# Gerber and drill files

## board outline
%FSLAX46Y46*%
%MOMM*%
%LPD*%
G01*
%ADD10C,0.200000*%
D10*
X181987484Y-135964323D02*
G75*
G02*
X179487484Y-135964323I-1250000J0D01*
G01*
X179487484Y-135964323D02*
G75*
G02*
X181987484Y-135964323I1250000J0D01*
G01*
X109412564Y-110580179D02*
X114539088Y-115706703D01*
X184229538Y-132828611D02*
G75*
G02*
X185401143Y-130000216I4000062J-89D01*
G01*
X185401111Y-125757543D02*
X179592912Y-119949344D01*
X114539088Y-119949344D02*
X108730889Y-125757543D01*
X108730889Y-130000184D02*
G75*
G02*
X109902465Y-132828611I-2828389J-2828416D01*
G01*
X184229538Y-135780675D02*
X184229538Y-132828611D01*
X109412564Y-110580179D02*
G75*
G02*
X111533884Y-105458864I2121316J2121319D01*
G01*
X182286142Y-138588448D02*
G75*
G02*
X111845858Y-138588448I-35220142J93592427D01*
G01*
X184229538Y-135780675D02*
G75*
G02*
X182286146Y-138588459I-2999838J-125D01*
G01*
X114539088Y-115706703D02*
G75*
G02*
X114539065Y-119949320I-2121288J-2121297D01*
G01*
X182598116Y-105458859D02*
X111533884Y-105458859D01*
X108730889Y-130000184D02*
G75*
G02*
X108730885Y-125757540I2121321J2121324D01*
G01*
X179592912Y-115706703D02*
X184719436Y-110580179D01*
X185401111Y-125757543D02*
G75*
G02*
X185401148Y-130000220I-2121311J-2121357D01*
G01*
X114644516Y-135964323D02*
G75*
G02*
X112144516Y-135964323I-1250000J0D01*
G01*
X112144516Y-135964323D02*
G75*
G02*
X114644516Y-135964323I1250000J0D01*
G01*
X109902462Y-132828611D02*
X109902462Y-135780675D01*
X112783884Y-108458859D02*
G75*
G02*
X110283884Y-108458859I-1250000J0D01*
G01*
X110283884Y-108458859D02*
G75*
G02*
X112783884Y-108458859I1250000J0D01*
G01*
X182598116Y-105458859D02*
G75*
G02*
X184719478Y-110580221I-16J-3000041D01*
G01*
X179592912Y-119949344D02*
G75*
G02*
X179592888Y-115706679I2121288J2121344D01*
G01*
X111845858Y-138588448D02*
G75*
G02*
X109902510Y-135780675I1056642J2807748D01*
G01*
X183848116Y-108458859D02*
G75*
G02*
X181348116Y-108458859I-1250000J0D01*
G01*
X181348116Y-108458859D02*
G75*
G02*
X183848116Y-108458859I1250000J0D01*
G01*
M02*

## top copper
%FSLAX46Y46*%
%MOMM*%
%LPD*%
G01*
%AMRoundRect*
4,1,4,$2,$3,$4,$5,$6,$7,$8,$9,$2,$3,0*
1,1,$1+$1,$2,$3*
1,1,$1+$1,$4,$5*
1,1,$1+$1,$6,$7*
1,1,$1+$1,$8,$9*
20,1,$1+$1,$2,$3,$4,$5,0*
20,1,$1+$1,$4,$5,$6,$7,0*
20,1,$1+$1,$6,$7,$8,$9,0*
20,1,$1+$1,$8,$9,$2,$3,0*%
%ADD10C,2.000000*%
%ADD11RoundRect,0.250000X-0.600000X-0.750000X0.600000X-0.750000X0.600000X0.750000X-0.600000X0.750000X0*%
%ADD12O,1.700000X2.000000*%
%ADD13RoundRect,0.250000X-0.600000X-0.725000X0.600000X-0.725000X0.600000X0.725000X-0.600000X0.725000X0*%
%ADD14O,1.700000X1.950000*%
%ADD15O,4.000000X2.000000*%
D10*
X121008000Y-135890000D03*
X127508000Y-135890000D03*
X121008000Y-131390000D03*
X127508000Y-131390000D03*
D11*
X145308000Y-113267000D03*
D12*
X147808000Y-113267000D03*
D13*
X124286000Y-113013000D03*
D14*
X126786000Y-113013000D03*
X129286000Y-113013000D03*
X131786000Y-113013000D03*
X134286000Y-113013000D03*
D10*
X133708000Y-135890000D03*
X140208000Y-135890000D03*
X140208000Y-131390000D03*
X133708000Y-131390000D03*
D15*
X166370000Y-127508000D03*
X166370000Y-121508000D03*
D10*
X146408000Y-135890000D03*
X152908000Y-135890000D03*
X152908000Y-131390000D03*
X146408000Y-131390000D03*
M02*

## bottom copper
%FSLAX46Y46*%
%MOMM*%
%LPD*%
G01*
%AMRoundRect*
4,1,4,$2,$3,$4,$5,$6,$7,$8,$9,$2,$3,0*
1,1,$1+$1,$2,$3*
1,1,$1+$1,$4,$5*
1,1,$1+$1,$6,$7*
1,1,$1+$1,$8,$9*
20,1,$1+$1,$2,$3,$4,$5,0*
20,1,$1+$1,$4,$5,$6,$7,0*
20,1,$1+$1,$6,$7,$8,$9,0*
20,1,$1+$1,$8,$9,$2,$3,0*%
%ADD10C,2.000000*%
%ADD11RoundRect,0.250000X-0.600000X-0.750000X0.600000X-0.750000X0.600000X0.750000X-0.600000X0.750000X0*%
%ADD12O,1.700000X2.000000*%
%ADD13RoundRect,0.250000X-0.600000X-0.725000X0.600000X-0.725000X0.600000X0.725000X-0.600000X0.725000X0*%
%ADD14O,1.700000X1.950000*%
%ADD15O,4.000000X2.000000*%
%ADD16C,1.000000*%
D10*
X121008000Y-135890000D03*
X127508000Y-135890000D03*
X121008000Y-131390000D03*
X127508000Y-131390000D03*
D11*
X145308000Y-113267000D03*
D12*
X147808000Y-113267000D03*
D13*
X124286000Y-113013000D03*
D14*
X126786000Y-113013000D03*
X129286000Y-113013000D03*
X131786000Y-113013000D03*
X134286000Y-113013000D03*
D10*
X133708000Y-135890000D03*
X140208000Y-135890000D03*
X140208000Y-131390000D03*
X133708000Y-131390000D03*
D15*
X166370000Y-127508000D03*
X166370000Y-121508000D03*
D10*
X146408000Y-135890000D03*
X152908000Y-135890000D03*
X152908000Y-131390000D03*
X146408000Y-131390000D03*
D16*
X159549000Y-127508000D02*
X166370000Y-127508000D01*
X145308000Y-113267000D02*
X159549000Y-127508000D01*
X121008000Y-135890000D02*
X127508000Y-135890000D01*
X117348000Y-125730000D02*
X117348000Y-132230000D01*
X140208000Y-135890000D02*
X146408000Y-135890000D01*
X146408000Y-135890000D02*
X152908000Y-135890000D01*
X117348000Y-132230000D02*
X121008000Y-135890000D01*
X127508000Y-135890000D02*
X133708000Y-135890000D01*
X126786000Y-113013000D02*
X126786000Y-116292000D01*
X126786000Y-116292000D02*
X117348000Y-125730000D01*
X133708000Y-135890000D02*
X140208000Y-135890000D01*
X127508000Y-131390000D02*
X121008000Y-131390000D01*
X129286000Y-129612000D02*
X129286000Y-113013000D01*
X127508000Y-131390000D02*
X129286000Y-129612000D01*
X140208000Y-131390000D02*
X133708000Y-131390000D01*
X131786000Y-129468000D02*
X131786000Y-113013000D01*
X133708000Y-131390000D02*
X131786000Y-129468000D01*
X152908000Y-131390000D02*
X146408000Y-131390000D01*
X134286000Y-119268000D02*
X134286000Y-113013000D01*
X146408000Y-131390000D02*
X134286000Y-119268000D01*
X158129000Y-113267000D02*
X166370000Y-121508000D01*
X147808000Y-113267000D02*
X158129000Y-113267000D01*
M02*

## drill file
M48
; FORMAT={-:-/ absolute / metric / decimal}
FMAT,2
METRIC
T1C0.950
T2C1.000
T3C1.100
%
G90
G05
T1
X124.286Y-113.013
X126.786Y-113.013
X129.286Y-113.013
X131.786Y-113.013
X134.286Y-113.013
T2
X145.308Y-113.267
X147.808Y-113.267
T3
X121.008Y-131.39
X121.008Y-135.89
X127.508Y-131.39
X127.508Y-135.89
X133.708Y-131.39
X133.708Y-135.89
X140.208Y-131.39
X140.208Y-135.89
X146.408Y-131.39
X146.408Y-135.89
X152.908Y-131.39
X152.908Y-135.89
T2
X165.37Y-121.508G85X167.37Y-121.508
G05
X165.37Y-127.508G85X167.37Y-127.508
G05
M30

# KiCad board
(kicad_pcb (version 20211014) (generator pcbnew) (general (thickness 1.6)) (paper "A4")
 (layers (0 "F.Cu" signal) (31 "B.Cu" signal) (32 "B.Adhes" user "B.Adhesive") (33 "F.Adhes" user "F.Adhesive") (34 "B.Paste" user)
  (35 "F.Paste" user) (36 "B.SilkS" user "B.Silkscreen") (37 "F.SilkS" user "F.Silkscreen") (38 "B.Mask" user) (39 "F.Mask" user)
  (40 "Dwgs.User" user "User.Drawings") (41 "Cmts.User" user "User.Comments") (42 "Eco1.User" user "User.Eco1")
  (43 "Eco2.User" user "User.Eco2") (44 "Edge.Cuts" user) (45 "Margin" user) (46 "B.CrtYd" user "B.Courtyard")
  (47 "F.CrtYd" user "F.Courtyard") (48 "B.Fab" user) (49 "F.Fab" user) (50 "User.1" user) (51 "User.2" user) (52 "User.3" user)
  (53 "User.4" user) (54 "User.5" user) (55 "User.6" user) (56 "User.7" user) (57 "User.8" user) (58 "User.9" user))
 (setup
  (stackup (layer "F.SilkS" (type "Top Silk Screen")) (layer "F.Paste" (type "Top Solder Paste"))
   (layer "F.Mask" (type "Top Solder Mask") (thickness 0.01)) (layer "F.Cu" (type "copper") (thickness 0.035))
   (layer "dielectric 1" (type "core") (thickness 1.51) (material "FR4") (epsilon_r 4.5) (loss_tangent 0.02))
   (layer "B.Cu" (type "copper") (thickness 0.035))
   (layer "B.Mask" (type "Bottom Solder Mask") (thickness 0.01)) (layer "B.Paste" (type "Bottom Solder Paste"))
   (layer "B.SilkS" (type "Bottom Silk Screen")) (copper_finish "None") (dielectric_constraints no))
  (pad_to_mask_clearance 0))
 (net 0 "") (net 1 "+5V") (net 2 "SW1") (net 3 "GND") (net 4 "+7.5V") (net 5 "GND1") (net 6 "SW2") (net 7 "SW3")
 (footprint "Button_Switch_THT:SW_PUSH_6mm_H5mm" (layer "F.Cu") (at 127.508 135.89 180)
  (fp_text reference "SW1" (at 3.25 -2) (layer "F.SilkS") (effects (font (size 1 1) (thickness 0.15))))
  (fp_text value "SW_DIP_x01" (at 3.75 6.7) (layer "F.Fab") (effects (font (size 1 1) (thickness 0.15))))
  (pad "1" thru_hole circle (at 6.5 0 270) (size 2 2) (drill 1.1) (layers *.Cu *.Mask) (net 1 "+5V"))
  (pad "1" thru_hole circle (at 0 0 270) (size 2 2) (drill 1.1) (layers *.Cu *.Mask) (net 1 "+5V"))
  (pad "2" thru_hole circle (at 6.5 4.5 270) (size 2 2) (drill 1.1) (layers *.Cu *.Mask) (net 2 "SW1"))
  (pad "2" thru_hole circle (at 0 4.5 270) (size 2 2) (drill 1.1) (layers *.Cu *.Mask) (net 2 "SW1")))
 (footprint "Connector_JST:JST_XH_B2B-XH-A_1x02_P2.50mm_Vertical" (layer "F.Cu") (at 145.308 113.267)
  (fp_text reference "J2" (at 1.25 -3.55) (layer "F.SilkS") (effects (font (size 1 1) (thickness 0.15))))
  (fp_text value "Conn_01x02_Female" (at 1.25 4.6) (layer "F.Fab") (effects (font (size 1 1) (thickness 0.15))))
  (pad "1" thru_hole roundrect (at 0 0) (size 1.7 2) (drill 1) (layers *.Cu *.Mask) (roundrect_rratio 0.1470588235) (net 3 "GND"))
  (pad "2" thru_hole oval (at 2.5 0) (size 1.7 2) (drill 1) (layers *.Cu *.Mask) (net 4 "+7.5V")))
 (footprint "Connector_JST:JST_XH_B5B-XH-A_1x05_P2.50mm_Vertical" (layer "F.Cu") (at 124.286 113.013)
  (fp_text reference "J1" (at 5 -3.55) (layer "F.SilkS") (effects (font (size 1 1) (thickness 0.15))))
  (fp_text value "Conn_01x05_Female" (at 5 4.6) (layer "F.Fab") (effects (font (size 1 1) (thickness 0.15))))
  (pad "1" thru_hole roundrect (at 0 0) (size 1.7 1.95) (drill 0.95) (layers *.Cu *.Mask) (roundrect_rratio 0.1470588235) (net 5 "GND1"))
  (pad "2" thru_hole oval (at 2.5 0) (size 1.7 1.95) (drill 0.95) (layers *.Cu *.Mask) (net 1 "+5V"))
  (pad "3" thru_hole oval (at 5 0) (size 1.7 1.95) (drill 0.95) (layers *.Cu *.Mask) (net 2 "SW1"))
  (pad "4" thru_hole oval (at 7.5 0) (size 1.7 1.95) (drill 0.95) (layers *.Cu *.Mask) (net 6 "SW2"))
  (pad "5" thru_hole oval (at 10 0) (size 1.7 1.95) (drill 0.95) (layers *.Cu *.Mask) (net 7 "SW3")))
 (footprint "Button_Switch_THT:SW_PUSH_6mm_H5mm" (layer "F.Cu") (at 140.208 135.89 180)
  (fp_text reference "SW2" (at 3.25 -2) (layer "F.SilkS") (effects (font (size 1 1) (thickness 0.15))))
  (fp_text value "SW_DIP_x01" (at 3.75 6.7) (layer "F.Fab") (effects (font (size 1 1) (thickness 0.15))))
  (pad "1" thru_hole circle (at 6.5 0 270) (size 2 2) (drill 1.1) (layers *.Cu *.Mask) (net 1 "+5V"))
  (pad "1" thru_hole circle (at 0 0 270) (size 2 2) (drill 1.1) (layers *.Cu *.Mask) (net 1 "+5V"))
  (pad "2" thru_hole circle (at 0 4.5 270) (size 2 2) (drill 1.1) (layers *.Cu *.Mask) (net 6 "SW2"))
  (pad "2" thru_hole circle (at 6.5 4.5 270) (size 2 2) (drill 1.1) (layers *.Cu *.Mask) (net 6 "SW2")))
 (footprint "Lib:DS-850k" (layer "F.Cu") (at 166.37 127.508 -90)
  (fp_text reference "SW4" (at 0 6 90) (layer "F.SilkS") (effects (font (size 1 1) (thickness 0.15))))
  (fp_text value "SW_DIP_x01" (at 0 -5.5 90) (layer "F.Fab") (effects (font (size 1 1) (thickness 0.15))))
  (pad "1" thru_hole oval locked (at 0 0) (size 4 2) (drill oval 3 1) (layers *.Cu *.Mask) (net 3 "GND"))
  (pad "2" thru_hole oval locked (at -6 0) (size 4 2) (drill oval 3 1) (layers *.Cu *.Mask) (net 4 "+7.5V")))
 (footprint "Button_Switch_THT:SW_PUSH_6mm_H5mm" (layer "F.Cu") (at 152.908 135.89 180)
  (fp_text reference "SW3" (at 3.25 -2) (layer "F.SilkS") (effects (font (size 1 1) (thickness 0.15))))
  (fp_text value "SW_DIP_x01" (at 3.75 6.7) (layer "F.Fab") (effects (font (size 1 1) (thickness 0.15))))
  (pad "1" thru_hole circle (at 6.5 0 270) (size 2 2) (drill 1.1) (layers *.Cu *.Mask) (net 1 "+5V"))
  (pad "1" thru_hole circle (at 0 0 270) (size 2 2) (drill 1.1) (layers *.Cu *.Mask) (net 1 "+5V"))
  (pad "2" thru_hole circle (at 0 4.5 270) (size 2 2) (drill 1.1) (layers *.Cu *.Mask) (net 7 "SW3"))
  (pad "2" thru_hole circle (at 6.5 4.5 270) (size 2 2) (drill 1.1) (layers *.Cu *.Mask) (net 7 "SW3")))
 (gr_circle (center 180.737484 135.964323) (end 181.987484 135.964323) (layer "Edge.Cuts") (width 0.2) (fill none))
 (gr_line (start 109.412564 110.580179) (end 114.539088 115.706703) (layer "Edge.Cuts") (width 0.2))
 (gr_arc (start 184.229538 132.828611) (mid 184.534027 131.297882) (end 185.401111 130.000184) (layer "Edge.Cuts") (width 0.2))
 (gr_line (start 185.401111 125.757543) (end 179.592912 119.949344) (layer "Edge.Cuts") (width 0.2))
 (gr_line (start 114.539088 119.949344) (end 108.730889 125.757543) (layer "Edge.Cuts") (width 0.2))
 (gr_arc (start 108.730889 130.000184) (mid 109.59798 131.297877) (end 109.902462 132.828611) (layer "Edge.Cuts") (width 0.2))
 (gr_line (start 184.229538 135.780675) (end 184.229538 132.828611) (layer "Edge.Cuts") (width 0.2))
 (gr_arc (start 109.412564 110.580179) (mid 108.762246 107.310809) (end 111.533884 105.458859) (layer "Edge.Cuts") (width 0.2))
 (gr_arc (start 182.286142 138.588448) (mid 147.066 144.996025) (end 111.845858 138.588448) (layer "Edge.Cuts") (width 0.2))
 (gr_arc (start 184.229538 135.780675) (mid 183.696321 137.488069) (end 182.286142 138.588448) (layer "Edge.Cuts") (width 0.2))
 (gr_arc (start 114.539088 115.706703) (mid 115.417768 117.828024) (end 114.539088 119.949344) (layer "Edge.Cuts") (width 0.2))
 (gr_line (start 182.598116 105.458859) (end 111.533884 105.458859) (layer "Edge.Cuts") (width 0.2))
 (gr_arc (start 108.730889 130.000184) (mid 107.852209 127.878864) (end 108.730889 125.757543) (layer "Edge.Cuts") (width 0.2))
 (gr_line (start 179.592912 115.706703) (end 184.719436 110.580179) (layer "Edge.Cuts") (width 0.2))
 (gr_arc (start 185.401111 125.757543) (mid 186.279792 127.878864) (end 185.401111 130.000184) (layer "Edge.Cuts") (width 0.2))
 (gr_circle (center 113.394516 135.964323) (end 114.644516 135.964323) (layer "Edge.Cuts") (width 0.2) (fill none))
 (gr_line (start 109.902462 132.828611) (end 109.902462 135.780675) (layer "Edge.Cuts") (width 0.2))
 (gr_circle (center 111.533884 108.458859) (end 112.783884 108.458859) (layer "Edge.Cuts") (width 0.2) (fill none))
 (gr_arc (start 182.598116 105.458859) (mid 185.369755 107.310807) (end 184.719436 110.580179) (layer "Edge.Cuts") (width 0.2))
 (gr_arc (start 179.592912 119.949344) (mid 178.714233 117.828024) (end 179.592912 115.706703) (layer "Edge.Cuts") (width 0.2))
 (gr_arc (start 111.845858 138.588448) (mid 110.435702 137.48804) (end 109.902462 135.780675) (layer "Edge.Cuts") (width 0.2))
 (gr_circle (center 182.598116 108.458859) (end 183.848116 108.458859) (layer "Edge.Cuts") (width 0.2) (fill none))
 (segment (start 159.549 127.508) (end 166.37 127.508) (width 1) (layer "B.Cu") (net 3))
 (segment (start 145.308 113.267) (end 159.549 127.508) (width 1) (layer "B.Cu") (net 3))
 (segment (start 121.008 135.89) (end 127.508 135.89) (width 1) (layer "B.Cu") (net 1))
 (segment (start 117.348 125.73) (end 117.348 132.23) (width 1) (layer "B.Cu") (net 1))
 (segment (start 140.208 135.89) (end 146.408 135.89) (width 1) (layer "B.Cu") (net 1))
 (segment (start 146.408 135.89) (end 152.908 135.89) (width 1) (layer "B.Cu") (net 1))
 (segment (start 117.348 132.23) (end 121.008 135.89) (width 1) (layer "B.Cu") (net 1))
 (segment (start 127.508 135.89) (end 133.708 135.89) (width 1) (layer "B.Cu") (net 1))
 (segment (start 126.786 113.013) (end 126.786 116.292) (width 1) (layer "B.Cu") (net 1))
 (segment (start 126.786 116.292) (end 117.348 125.73) (width 1) (layer "B.Cu") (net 1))
 (segment (start 133.708 135.89) (end 140.208 135.89) (width 1) (layer "B.Cu") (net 1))
 (segment (start 127.508 131.39) (end 121.008 131.39) (width 1) (layer "B.Cu") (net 2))
 (segment (start 129.286 129.612) (end 129.286 113.013) (width 1) (layer "B.Cu") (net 2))
 (segment (start 127.508 131.39) (end 129.286 129.612) (width 1) (layer "B.Cu") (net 2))
 (segment (start 140.208 131.39) (end 133.708 131.39) (width 1) (layer "B.Cu") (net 6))
 (segment (start 131.786 129.468) (end 131.786 113.013) (width 1) (layer "B.Cu") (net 6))
 (segment (start 133.708 131.39) (end 131.786 129.468) (width 1) (layer "B.Cu") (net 6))
 (segment (start 152.908 131.39) (end 146.408 131.39) (width 1) (layer "B.Cu") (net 7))
 (segment (start 134.286 119.268) (end 134.286 113.013) (width 1) (layer "B.Cu") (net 7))
 (segment (start 146.408 131.39) (end 134.286 119.268) (width 1) (layer "B.Cu") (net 7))
 (segment (start 158.129 113.267) (end 166.37 121.508) (width 1) (layer "B.Cu") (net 4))
 (segment (start 147.808 113.267) (end 158.129 113.267) (width 1) (layer "B.Cu") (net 4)))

